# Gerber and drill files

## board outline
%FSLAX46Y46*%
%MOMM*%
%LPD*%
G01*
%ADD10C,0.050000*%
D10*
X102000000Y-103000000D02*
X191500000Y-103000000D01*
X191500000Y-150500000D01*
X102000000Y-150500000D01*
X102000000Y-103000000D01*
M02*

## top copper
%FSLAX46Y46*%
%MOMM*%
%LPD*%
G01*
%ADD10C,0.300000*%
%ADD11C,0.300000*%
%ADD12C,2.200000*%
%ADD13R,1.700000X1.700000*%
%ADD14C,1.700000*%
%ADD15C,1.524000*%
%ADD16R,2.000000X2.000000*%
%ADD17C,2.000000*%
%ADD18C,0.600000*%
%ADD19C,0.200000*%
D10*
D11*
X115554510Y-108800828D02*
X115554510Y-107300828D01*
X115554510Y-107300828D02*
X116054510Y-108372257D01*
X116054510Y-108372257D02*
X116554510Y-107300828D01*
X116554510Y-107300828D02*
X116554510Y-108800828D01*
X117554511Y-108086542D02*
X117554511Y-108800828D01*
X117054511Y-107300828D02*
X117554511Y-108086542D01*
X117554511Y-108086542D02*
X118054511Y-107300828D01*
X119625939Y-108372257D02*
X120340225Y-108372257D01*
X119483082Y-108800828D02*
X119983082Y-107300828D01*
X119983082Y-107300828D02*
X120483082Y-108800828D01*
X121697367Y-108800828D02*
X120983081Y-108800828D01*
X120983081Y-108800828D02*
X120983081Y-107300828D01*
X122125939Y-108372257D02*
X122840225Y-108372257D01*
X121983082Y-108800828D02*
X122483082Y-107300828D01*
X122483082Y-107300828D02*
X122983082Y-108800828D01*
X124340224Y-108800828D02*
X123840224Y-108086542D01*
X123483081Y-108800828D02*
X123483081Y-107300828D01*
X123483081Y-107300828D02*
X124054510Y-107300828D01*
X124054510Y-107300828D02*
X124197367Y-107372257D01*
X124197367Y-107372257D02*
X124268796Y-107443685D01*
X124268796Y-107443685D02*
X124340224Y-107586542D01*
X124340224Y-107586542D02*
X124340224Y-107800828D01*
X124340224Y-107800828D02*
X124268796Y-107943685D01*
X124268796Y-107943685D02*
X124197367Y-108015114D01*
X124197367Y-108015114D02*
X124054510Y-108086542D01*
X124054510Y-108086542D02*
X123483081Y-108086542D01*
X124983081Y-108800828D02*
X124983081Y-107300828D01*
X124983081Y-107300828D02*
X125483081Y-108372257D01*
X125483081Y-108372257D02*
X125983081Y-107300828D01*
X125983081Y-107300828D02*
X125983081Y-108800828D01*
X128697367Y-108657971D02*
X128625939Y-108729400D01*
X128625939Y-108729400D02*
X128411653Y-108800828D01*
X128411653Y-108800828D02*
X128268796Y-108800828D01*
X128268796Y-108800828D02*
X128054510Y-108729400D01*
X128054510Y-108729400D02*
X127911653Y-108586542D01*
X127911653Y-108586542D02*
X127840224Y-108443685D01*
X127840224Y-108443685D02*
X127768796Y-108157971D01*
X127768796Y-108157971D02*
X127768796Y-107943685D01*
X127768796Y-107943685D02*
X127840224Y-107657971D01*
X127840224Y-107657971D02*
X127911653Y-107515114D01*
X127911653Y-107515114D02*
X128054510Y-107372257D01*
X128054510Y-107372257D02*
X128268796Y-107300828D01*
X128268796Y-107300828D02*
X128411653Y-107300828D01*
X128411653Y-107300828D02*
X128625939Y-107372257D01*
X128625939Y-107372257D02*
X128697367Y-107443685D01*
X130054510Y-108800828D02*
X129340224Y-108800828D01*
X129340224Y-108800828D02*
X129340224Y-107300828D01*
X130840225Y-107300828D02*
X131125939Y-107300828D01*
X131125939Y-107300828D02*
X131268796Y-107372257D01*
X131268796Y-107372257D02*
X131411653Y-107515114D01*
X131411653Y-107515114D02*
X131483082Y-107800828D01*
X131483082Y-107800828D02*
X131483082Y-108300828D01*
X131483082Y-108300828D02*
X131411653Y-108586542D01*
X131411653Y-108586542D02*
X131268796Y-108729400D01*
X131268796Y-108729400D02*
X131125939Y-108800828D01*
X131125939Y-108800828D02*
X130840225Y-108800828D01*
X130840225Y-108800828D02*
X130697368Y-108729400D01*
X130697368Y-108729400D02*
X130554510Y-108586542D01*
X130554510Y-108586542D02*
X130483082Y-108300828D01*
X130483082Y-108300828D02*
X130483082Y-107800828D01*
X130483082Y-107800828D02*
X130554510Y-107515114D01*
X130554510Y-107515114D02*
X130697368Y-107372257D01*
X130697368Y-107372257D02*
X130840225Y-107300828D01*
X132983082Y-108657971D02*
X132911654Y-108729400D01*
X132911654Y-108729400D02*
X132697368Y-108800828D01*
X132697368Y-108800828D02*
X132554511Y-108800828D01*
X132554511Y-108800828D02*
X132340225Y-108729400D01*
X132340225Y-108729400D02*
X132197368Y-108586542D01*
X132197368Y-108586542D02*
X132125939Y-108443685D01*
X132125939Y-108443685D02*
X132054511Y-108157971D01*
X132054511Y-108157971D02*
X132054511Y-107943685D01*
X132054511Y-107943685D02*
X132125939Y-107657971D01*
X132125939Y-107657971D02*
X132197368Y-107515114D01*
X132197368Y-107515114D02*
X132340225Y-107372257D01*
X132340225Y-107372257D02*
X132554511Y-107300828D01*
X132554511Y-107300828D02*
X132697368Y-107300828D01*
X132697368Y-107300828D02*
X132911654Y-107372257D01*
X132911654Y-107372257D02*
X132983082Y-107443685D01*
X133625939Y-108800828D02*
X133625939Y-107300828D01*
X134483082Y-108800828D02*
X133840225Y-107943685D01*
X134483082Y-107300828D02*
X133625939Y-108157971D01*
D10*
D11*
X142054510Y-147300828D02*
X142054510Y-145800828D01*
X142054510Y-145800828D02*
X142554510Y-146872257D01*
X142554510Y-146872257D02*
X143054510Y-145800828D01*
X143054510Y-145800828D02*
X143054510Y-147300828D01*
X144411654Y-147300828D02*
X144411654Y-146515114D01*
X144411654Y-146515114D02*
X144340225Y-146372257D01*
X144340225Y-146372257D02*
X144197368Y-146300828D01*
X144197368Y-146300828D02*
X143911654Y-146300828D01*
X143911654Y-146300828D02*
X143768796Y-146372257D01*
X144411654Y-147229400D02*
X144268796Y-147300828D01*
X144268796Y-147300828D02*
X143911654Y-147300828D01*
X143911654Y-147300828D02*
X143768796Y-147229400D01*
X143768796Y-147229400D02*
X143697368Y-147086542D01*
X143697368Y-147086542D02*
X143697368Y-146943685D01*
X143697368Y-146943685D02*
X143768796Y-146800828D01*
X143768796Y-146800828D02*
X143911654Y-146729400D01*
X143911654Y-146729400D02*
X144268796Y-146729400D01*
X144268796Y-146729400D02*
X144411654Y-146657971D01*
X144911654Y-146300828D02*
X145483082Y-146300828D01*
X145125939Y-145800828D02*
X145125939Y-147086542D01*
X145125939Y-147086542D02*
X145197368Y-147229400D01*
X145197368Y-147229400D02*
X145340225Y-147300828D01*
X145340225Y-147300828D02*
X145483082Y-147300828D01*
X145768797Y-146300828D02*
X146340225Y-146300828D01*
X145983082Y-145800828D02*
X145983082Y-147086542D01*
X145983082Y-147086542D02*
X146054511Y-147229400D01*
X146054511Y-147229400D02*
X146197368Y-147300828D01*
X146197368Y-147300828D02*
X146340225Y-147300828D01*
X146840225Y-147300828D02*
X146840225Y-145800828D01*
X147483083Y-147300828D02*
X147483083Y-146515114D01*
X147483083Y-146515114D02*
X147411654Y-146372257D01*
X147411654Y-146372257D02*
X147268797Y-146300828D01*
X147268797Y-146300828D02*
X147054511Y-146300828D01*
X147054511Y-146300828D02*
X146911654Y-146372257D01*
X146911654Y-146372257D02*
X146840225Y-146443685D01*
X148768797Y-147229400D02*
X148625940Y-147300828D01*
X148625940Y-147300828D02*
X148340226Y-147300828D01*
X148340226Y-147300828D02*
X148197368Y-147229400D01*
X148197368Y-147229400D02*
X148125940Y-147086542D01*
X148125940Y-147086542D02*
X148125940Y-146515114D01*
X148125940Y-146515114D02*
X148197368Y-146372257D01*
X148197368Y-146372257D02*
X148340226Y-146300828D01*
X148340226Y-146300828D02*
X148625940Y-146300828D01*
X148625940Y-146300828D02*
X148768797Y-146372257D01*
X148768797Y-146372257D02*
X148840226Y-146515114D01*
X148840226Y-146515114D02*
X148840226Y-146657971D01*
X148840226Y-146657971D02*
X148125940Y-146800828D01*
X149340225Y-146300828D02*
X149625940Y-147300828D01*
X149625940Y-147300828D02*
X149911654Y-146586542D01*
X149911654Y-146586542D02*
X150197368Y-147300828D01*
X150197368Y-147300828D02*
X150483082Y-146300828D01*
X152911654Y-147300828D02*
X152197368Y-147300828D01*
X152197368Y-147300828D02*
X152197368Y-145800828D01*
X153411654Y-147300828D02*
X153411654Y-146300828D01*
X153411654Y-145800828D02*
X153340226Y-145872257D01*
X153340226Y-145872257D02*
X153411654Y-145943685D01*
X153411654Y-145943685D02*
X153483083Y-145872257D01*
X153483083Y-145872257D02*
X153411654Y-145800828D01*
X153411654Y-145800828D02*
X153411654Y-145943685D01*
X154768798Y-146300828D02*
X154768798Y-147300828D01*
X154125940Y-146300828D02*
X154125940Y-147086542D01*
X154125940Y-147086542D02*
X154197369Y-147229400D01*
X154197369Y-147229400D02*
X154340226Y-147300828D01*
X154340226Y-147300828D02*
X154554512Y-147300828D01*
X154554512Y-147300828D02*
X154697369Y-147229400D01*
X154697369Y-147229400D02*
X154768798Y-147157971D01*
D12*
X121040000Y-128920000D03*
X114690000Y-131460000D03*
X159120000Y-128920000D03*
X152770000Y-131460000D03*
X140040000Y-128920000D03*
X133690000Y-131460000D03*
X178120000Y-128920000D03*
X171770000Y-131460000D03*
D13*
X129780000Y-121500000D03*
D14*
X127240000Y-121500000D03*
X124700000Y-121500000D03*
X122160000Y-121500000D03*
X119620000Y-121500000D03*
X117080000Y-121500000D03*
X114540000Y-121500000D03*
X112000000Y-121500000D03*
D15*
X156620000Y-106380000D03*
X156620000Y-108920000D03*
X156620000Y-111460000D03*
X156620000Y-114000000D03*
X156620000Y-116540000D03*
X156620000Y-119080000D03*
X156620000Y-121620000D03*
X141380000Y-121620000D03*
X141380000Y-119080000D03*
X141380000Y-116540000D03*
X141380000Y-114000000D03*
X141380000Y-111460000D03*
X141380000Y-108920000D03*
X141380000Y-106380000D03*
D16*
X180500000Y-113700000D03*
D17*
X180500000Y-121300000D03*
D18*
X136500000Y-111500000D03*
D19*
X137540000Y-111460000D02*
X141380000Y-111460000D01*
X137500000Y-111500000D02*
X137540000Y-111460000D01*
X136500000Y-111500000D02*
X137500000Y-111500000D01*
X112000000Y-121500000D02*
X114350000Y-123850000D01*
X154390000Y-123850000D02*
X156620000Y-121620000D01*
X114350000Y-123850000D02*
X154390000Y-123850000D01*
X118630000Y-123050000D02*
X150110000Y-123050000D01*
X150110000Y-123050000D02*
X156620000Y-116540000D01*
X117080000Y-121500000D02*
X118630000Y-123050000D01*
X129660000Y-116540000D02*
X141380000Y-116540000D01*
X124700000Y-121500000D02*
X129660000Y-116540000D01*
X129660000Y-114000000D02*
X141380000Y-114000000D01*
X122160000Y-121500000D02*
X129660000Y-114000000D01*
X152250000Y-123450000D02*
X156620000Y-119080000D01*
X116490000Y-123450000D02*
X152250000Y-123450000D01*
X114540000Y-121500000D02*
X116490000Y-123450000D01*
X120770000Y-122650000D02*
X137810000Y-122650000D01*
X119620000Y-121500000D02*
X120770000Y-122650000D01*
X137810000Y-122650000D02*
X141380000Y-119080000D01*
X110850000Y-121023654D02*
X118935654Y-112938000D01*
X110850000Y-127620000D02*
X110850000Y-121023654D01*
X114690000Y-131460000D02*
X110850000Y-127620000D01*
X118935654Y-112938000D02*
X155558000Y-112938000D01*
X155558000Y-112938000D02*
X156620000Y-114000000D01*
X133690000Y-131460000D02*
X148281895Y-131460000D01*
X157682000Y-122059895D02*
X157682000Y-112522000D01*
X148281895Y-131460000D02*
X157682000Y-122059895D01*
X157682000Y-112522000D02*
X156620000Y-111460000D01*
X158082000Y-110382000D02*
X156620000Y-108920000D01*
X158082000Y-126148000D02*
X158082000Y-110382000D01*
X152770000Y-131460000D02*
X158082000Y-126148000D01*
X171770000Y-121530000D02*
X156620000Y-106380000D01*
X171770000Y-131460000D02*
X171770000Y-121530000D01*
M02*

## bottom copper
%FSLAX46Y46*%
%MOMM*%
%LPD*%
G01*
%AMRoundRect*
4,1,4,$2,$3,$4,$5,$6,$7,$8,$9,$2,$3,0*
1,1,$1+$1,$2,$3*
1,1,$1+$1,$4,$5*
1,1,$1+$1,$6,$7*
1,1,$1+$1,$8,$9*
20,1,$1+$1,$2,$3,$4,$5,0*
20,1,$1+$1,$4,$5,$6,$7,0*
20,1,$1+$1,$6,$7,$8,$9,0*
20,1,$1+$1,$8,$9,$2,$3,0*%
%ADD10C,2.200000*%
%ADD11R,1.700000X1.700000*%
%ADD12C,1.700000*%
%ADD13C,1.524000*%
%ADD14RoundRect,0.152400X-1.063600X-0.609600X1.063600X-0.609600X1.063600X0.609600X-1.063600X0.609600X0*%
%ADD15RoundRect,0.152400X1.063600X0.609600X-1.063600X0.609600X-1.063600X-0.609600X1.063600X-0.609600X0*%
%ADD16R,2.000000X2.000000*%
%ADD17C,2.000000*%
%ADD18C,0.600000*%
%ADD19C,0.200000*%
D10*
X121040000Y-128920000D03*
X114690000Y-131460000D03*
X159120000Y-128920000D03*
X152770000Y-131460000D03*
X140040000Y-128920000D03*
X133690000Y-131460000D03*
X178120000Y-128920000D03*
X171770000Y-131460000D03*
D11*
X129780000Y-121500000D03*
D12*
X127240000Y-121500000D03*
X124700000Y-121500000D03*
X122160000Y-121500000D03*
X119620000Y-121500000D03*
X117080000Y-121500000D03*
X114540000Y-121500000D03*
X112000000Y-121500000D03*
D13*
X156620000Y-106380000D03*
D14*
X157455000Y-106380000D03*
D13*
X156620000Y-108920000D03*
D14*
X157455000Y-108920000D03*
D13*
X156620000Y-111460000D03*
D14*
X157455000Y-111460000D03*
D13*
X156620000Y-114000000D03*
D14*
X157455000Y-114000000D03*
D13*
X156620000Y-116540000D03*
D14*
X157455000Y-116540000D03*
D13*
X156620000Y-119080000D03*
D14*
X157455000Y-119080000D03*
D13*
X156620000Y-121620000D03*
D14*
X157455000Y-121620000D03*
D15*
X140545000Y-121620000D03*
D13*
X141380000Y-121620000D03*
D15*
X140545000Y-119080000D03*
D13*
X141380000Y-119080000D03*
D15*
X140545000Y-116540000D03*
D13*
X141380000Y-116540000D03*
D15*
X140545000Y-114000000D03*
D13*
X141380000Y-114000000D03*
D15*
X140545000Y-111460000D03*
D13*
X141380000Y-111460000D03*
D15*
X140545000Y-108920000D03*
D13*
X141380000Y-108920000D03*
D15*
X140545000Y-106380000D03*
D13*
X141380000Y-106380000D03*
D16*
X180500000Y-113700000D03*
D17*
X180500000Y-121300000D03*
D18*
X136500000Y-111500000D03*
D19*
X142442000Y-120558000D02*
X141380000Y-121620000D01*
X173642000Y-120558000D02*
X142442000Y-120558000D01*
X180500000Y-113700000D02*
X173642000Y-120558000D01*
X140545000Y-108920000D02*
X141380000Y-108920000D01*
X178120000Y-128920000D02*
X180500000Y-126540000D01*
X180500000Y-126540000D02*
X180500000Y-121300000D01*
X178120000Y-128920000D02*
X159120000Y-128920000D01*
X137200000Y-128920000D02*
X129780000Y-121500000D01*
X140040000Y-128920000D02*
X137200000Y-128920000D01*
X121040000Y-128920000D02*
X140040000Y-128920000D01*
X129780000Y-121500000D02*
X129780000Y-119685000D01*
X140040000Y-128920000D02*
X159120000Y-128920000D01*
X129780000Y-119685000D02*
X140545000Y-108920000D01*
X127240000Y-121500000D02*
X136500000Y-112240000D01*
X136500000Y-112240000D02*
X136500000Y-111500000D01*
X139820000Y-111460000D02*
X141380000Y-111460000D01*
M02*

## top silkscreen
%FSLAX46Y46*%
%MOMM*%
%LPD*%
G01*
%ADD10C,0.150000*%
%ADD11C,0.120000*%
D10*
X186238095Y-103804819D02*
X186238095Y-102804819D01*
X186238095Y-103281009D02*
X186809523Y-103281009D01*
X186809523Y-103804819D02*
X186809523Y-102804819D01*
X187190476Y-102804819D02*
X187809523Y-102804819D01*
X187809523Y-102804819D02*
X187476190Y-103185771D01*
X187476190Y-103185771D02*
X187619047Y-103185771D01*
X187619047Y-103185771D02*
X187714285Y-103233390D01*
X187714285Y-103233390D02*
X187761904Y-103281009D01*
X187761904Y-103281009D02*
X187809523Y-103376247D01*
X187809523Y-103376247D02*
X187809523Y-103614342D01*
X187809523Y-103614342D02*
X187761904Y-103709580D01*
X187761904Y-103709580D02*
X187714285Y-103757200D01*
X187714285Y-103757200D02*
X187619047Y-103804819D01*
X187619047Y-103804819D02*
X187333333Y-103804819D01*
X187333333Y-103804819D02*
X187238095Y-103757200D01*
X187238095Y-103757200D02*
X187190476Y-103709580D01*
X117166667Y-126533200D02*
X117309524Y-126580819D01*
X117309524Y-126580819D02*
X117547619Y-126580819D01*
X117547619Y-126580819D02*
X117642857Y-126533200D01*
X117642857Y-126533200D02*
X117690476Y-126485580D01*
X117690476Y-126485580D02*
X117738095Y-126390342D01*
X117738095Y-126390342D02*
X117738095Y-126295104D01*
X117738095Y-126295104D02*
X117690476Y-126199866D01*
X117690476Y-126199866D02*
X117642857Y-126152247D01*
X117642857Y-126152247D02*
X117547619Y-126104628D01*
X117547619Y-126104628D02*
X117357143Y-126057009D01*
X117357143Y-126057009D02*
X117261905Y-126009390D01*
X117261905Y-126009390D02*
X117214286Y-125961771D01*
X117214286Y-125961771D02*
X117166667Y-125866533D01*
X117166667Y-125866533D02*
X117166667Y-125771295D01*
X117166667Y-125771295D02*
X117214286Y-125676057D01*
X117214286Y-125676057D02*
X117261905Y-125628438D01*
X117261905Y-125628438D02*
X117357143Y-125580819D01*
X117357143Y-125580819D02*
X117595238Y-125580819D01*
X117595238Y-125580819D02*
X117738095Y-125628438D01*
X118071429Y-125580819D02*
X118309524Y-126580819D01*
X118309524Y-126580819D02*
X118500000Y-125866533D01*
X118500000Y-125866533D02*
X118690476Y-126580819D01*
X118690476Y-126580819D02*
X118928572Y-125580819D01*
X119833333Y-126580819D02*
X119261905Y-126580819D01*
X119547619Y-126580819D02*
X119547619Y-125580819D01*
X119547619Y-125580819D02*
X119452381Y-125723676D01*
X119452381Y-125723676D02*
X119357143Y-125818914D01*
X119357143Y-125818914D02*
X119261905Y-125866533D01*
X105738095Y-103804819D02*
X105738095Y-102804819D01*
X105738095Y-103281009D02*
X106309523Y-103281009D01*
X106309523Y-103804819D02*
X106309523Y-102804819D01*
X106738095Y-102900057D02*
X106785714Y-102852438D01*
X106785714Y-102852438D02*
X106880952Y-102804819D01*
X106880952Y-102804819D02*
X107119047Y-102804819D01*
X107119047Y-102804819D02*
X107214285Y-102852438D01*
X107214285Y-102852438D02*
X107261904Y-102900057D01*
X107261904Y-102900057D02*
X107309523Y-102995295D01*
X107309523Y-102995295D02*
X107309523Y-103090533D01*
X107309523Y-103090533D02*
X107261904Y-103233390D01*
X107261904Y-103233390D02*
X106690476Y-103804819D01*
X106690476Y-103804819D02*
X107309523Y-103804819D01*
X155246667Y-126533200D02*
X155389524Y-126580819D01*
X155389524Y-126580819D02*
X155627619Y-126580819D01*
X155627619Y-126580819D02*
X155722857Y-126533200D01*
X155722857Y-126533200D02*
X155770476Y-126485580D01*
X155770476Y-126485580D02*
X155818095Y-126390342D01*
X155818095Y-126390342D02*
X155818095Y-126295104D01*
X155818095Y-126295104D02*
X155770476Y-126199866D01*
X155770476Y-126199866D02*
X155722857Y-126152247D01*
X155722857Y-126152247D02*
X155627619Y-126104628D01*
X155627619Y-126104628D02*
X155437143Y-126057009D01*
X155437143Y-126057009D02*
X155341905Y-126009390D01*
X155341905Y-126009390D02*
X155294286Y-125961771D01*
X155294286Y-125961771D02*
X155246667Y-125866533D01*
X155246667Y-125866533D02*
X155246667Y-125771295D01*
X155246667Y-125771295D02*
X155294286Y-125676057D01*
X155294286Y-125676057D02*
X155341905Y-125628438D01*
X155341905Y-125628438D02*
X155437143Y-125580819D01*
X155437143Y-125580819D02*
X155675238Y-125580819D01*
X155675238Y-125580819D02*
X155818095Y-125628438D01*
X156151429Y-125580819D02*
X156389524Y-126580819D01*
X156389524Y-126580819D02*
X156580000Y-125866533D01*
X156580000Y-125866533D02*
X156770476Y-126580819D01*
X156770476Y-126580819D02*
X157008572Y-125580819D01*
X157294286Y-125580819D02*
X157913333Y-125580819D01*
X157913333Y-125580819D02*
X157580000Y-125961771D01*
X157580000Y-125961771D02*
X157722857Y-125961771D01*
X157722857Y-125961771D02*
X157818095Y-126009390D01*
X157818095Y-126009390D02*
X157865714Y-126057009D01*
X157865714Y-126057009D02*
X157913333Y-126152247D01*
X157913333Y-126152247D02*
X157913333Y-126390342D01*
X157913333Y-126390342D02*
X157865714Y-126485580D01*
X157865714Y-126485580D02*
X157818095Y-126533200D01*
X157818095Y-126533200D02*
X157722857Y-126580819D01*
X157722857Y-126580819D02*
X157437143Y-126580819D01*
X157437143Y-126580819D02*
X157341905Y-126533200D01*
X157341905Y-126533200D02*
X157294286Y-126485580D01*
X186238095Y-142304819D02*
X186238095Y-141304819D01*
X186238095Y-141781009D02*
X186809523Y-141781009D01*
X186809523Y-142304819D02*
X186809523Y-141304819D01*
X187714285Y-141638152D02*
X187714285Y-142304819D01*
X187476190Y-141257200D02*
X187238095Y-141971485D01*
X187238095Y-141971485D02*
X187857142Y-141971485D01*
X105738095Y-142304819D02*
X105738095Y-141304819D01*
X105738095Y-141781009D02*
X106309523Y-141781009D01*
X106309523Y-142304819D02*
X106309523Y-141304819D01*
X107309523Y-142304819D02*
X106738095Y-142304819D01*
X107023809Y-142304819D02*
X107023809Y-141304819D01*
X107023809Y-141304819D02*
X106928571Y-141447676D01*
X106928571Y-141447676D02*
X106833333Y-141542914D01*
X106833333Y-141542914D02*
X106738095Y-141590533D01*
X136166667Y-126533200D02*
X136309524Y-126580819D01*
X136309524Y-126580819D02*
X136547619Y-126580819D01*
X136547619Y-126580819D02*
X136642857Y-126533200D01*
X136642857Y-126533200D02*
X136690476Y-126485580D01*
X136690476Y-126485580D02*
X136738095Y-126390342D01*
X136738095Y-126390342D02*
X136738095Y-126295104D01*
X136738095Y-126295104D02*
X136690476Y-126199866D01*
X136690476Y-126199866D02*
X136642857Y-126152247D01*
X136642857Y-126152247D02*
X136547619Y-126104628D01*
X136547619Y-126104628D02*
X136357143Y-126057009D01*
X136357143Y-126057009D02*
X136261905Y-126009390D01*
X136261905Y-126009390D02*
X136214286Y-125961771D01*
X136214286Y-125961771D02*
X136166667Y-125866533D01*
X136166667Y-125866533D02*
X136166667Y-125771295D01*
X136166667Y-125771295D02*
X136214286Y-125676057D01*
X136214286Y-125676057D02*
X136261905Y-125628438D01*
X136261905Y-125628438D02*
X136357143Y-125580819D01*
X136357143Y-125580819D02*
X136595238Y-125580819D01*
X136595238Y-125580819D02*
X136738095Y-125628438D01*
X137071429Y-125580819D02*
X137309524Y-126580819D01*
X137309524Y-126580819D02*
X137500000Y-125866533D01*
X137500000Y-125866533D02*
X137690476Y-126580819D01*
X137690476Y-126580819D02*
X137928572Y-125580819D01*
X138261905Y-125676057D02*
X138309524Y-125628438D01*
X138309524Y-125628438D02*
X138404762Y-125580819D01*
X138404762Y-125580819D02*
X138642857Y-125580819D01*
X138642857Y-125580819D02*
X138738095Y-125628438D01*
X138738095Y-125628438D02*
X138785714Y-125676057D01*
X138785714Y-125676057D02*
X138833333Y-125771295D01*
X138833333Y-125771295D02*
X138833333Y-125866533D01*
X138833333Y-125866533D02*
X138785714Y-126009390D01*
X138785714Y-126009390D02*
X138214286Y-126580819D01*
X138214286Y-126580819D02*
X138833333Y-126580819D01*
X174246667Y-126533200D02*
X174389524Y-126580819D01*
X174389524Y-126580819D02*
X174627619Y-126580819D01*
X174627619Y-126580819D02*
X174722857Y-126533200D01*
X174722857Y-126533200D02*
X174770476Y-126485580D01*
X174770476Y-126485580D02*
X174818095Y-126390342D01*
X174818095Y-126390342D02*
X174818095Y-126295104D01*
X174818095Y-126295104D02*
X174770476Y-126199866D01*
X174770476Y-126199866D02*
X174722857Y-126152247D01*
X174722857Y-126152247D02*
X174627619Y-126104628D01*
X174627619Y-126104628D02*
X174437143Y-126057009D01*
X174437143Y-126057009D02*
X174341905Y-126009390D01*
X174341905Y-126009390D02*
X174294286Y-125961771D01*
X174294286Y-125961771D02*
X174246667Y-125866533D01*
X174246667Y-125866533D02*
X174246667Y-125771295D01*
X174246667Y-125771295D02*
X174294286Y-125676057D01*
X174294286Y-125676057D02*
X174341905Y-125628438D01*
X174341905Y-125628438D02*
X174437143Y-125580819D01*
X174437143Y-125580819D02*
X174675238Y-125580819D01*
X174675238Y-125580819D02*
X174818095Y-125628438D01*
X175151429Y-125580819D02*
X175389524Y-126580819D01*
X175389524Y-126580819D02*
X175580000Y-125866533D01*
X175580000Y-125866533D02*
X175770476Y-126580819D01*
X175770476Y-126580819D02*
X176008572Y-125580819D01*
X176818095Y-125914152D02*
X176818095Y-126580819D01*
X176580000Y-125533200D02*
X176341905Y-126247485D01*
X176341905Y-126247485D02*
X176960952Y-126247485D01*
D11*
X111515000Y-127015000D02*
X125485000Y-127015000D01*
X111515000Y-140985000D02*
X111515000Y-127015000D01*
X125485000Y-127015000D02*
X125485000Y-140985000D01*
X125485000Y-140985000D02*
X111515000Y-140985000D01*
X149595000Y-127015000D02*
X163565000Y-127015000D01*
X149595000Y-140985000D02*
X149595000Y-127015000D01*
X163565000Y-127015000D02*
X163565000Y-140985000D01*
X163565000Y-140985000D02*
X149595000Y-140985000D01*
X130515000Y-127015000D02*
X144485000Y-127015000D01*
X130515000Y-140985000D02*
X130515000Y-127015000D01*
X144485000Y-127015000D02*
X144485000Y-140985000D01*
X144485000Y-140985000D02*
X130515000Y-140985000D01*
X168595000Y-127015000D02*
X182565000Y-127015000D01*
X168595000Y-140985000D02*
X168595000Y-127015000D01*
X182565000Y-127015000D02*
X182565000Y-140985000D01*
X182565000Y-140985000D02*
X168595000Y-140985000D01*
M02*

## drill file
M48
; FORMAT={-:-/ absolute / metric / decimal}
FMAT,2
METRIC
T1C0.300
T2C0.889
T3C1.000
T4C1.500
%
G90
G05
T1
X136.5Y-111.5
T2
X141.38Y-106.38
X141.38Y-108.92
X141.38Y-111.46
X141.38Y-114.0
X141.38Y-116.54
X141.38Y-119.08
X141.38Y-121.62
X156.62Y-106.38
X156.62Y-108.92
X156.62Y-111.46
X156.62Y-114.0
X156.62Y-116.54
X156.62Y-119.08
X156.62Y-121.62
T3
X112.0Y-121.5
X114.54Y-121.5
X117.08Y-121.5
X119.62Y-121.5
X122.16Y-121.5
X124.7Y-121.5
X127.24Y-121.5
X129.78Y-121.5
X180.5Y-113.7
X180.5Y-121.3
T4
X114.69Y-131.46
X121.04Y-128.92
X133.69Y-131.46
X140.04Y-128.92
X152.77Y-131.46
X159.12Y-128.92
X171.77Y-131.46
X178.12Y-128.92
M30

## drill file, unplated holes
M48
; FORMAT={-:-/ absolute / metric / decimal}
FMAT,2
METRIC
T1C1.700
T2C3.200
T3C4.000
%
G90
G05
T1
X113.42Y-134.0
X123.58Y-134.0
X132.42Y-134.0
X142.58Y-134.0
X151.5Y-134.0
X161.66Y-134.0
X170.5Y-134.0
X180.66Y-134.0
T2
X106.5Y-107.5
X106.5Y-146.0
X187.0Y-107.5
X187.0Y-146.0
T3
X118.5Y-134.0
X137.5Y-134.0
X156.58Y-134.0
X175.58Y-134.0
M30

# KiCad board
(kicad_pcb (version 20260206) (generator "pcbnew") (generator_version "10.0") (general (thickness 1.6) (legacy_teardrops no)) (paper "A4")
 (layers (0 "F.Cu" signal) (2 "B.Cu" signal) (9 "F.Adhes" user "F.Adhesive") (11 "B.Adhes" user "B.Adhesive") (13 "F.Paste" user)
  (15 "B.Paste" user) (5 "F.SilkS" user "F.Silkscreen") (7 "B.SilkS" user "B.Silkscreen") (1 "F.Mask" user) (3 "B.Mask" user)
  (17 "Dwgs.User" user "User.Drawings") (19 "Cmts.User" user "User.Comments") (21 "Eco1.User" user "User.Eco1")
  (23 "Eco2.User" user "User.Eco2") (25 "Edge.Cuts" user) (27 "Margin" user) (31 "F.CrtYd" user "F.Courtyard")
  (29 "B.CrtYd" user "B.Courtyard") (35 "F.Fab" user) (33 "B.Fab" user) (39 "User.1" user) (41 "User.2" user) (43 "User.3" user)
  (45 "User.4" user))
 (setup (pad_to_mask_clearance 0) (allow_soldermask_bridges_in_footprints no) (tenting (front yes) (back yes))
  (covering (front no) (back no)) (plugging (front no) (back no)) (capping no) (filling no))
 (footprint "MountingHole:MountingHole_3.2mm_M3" (layer "F.Cu") (at 187 107.5)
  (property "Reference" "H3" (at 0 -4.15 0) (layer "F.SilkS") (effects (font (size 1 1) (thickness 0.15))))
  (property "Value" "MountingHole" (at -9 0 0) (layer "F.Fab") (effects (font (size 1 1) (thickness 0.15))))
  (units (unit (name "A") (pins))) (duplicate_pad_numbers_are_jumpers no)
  (pad "" np_thru_hole circle (at 0 0) (size 3.2 3.2) (drill 3.2) (layers "*.Cu" "*.Mask")))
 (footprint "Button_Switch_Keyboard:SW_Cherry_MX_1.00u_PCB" (layer "F.Cu") (at 121.04 128.92)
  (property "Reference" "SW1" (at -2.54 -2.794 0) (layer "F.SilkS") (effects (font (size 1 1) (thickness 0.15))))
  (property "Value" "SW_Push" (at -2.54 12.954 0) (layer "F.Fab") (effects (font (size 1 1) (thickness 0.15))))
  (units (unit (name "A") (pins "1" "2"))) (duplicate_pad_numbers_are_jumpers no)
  (fp_line (start -9.525 -1.905) (end 4.445 -1.905) (stroke (width 0.12) (type solid)) (layer "F.SilkS"))
  (fp_line (start -9.525 12.065) (end -9.525 -1.905) (stroke (width 0.12) (type solid)) (layer "F.SilkS"))
  (fp_line (start 4.445 -1.905) (end 4.445 12.065) (stroke (width 0.12) (type solid)) (layer "F.SilkS"))
  (fp_line (start 4.445 12.065) (end -9.525 12.065) (stroke (width 0.12) (type solid)) (layer "F.SilkS"))
  (pad "" np_thru_hole circle (at -7.62 5.08) (size 1.7 1.7) (drill 1.7) (layers "*.Cu" "*.Mask"))
  (pad "" np_thru_hole circle (at -2.54 5.08) (size 4 4) (drill 4) (layers "*.Cu" "*.Mask"))
  (pad "" np_thru_hole circle (at 2.54 5.08) (size 1.7 1.7) (drill 1.7) (layers "*.Cu" "*.Mask"))
  (pad "1" thru_hole circle (at 0 0) (size 2.2 2.2) (drill 1.5) (layers "*.Cu" "*.Mask") (remove_unused_layers no) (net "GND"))
  (pad "2" thru_hole circle (at -6.35 2.54) (size 2.2 2.2) (drill 1.5) (layers "*.Cu" "*.Mask") (remove_unused_layers no)
   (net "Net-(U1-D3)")))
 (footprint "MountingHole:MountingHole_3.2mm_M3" (layer "F.Cu") (at 106.5 107.5)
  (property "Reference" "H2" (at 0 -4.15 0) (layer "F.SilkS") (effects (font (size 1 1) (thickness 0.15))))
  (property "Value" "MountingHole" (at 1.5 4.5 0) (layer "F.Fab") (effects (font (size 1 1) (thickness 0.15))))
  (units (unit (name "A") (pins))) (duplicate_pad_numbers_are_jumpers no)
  (pad "" np_thru_hole circle (at 0 0) (size 3.2 3.2) (drill 3.2) (layers "*.Cu" "*.Mask")))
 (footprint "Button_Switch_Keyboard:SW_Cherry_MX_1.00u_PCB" (layer "F.Cu") (at 159.12 128.92)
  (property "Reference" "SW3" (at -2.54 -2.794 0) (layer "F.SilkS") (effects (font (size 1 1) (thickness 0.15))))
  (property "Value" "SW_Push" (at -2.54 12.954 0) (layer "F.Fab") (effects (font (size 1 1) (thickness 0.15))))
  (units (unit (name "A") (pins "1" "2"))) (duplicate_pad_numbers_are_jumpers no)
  (fp_line (start -9.525 -1.905) (end 4.445 -1.905) (stroke (width 0.12) (type solid)) (layer "F.SilkS"))
  (fp_line (start -9.525 12.065) (end -9.525 -1.905) (stroke (width 0.12) (type solid)) (layer "F.SilkS"))
  (fp_line (start 4.445 -1.905) (end 4.445 12.065) (stroke (width 0.12) (type solid)) (layer "F.SilkS"))
  (fp_line (start 4.445 12.065) (end -9.525 12.065) (stroke (width 0.12) (type solid)) (layer "F.SilkS"))
  (pad "" np_thru_hole circle (at -7.62 5.08) (size 1.7 1.7) (drill 1.7) (layers "*.Cu" "*.Mask"))
  (pad "" np_thru_hole circle (at -2.54 5.08) (size 4 4) (drill 4) (layers "*.Cu" "*.Mask"))
  (pad "" np_thru_hole circle (at 2.54 5.08) (size 1.7 1.7) (drill 1.7) (layers "*.Cu" "*.Mask"))
  (pad "1" thru_hole circle (at 0 0) (size 2.2 2.2) (drill 1.5) (layers "*.Cu" "*.Mask") (remove_unused_layers no) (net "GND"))
  (pad "2" thru_hole circle (at -6.35 2.54) (size 2.2 2.2) (drill 1.5) (layers "*.Cu" "*.Mask") (remove_unused_layers no)
   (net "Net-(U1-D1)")))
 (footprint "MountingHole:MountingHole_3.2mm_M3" (layer "F.Cu") (at 187 146)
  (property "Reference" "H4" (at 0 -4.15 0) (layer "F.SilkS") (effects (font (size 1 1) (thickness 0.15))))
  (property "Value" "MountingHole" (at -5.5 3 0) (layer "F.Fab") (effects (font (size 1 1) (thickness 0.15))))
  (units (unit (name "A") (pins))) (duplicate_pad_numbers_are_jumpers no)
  (pad "" np_thru_hole circle (at 0 0) (size 3.2 3.2) (drill 3.2) (layers "*.Cu" "*.Mask")))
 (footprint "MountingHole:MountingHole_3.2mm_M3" (layer "F.Cu") (at 106.5 146)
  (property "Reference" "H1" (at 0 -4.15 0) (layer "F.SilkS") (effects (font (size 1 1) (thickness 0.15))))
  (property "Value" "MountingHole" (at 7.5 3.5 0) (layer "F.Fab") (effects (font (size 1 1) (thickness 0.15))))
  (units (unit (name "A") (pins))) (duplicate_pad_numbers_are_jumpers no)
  (pad "" np_thru_hole circle (at 0 0) (size 3.2 3.2) (drill 3.2) (layers "*.Cu" "*.Mask")))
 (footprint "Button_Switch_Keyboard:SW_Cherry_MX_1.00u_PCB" (layer "F.Cu") (at 140.04 128.92)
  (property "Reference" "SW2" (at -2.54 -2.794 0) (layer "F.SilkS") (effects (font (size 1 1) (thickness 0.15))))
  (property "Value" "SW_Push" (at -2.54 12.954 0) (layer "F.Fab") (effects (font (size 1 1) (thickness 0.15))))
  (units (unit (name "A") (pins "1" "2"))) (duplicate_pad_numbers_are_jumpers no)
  (fp_line (start -9.525 -1.905) (end 4.445 -1.905) (stroke (width 0.12) (type solid)) (layer "F.SilkS"))
  (fp_line (start -9.525 12.065) (end -9.525 -1.905) (stroke (width 0.12) (type solid)) (layer "F.SilkS"))
  (fp_line (start 4.445 -1.905) (end 4.445 12.065) (stroke (width 0.12) (type solid)) (layer "F.SilkS"))
  (fp_line (start 4.445 12.065) (end -9.525 12.065) (stroke (width 0.12) (type solid)) (layer "F.SilkS"))
  (pad "" np_thru_hole circle (at -7.62 5.08) (size 1.7 1.7) (drill 1.7) (layers "*.Cu" "*.Mask"))
  (pad "" np_thru_hole circle (at -2.54 5.08) (size 4 4) (drill 4) (layers "*.Cu" "*.Mask"))
  (pad "" np_thru_hole circle (at 2.54 5.08) (size 1.7 1.7) (drill 1.7) (layers "*.Cu" "*.Mask"))
  (pad "1" thru_hole circle (at 0 0) (size 2.2 2.2) (drill 1.5) (layers "*.Cu" "*.Mask") (remove_unused_layers no) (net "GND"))
  (pad "2" thru_hole circle (at -6.35 2.54) (size 2.2 2.2) (drill 1.5) (layers "*.Cu" "*.Mask") (remove_unused_layers no)
   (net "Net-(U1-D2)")))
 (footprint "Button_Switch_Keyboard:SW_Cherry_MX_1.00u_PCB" (layer "F.Cu") (at 178.12 128.92)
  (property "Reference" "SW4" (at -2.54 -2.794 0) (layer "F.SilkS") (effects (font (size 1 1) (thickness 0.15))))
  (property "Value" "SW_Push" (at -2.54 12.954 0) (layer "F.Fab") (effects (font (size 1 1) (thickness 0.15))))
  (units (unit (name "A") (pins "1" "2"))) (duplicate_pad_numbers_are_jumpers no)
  (fp_line (start -9.525 -1.905) (end 4.445 -1.905) (stroke (width 0.12) (type solid)) (layer "F.SilkS"))
  (fp_line (start -9.525 12.065) (end -9.525 -1.905) (stroke (width 0.12) (type solid)) (layer "F.SilkS"))
  (fp_line (start 4.445 -1.905) (end 4.445 12.065) (stroke (width 0.12) (type solid)) (layer "F.SilkS"))
  (fp_line (start 4.445 12.065) (end -9.525 12.065) (stroke (width 0.12) (type solid)) (layer "F.SilkS"))
  (pad "" np_thru_hole circle (at -7.62 5.08) (size 1.7 1.7) (drill 1.7) (layers "*.Cu" "*.Mask"))
  (pad "" np_thru_hole circle (at -2.54 5.08) (size 4 4) (drill 4) (layers "*.Cu" "*.Mask"))
  (pad "" np_thru_hole circle (at 2.54 5.08) (size 1.7 1.7) (drill 1.7) (layers "*.Cu" "*.Mask"))
  (pad "1" thru_hole circle (at 0 0) (size 2.2 2.2) (drill 1.5) (layers "*.Cu" "*.Mask") (remove_unused_layers no) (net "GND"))
  (pad "2" thru_hole circle (at -6.35 2.54) (size 2.2 2.2) (drill 1.5) (layers "*.Cu" "*.Mask") (remove_unused_layers no)
   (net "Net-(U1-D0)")))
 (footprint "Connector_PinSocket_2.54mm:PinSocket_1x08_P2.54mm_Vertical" (layer "B.Cu") (at 129.78 121.5 90)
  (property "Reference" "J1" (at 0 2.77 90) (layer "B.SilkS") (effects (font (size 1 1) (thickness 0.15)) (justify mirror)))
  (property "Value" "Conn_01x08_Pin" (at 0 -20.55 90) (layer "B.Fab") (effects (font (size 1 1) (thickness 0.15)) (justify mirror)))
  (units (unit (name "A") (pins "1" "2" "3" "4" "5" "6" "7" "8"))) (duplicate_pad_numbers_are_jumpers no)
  (pad "1" thru_hole rect (at 0 0 90) (size 1.7 1.7) (drill 1) (layers "*.Cu" "*.Mask") (remove_unused_layers no) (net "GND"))
  (pad "2" thru_hole circle (at 0 -2.54 90) (size 1.7 1.7) (drill 1) (layers "*.Cu" "*.Mask") (remove_unused_layers no) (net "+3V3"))
  (pad "3" thru_hole circle (at 0 -5.08 90) (size 1.7 1.7) (drill 1) (layers "*.Cu" "*.Mask") (remove_unused_layers no) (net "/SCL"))
  (pad "4" thru_hole circle (at 0 -7.62 90) (size 1.7 1.7) (drill 1) (layers "*.Cu" "*.Mask") (remove_unused_layers no) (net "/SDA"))
  (pad "5" thru_hole circle (at 0 -10.16 90) (size 1.7 1.7) (drill 1) (layers "*.Cu" "*.Mask") (remove_unused_layers no) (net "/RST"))
  (pad "6" thru_hole circle (at 0 -12.7 90) (size 1.7 1.7) (drill 1) (layers "*.Cu" "*.Mask") (remove_unused_layers no) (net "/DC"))
  (pad "7" thru_hole circle (at 0 -15.24 90) (size 1.7 1.7) (drill 1) (layers "*.Cu" "*.Mask") (remove_unused_layers no) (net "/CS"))
  (pad "8" thru_hole circle (at 0 -17.78 90) (size 1.7 1.7) (drill 1) (layers "*.Cu" "*.Mask") (remove_unused_layers no) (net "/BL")))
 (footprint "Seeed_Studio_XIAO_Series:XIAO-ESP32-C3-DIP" (layer "B.Cu") (at 149 114 90)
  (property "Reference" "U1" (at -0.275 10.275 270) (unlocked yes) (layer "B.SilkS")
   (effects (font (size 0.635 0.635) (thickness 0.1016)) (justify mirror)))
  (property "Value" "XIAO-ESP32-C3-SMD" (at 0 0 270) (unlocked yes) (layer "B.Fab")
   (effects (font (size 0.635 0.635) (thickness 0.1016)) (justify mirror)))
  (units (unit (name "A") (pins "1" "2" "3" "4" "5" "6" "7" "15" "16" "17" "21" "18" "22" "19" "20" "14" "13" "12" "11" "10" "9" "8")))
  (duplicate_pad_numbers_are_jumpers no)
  (pad "1" thru_hole circle (at 7.62 7.62) (size 1.524 1.524) (drill 0.889) (layers "*.Cu" "*.Mask") (remove_unused_layers no)
   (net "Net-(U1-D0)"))
  (pad "1" smd roundrect (at 7.62 8.455) (size 2.432 1.524) (layers "B.Cu" "B.Mask") (roundrect_rratio 0.1) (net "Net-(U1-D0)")
   (thermal_bridge_angle 45))
  (pad "2" thru_hole circle (at 5.08 7.62) (size 1.524 1.524) (drill 0.889) (layers "*.Cu" "*.Mask") (remove_unused_layers no)
   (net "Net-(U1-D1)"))
  (pad "2" smd roundrect (at 5.08 8.455) (size 2.432 1.524) (layers "B.Cu" "B.Mask") (roundrect_rratio 0.1) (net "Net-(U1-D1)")
   (thermal_bridge_angle 45))
  (pad "3" thru_hole circle (at 2.54 7.62) (size 1.524 1.524) (drill 0.889) (layers "*.Cu" "*.Mask") (remove_unused_layers no)
   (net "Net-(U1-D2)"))
  (pad "3" smd roundrect (at 2.54 8.455) (size 2.432 1.524) (layers "B.Cu" "B.Mask") (roundrect_rratio 0.1) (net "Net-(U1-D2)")
   (thermal_bridge_angle 45))
  (pad "4" thru_hole circle (at 0 7.62) (size 1.524 1.524) (drill 0.889) (layers "*.Cu" "*.Mask") (remove_unused_layers no)
   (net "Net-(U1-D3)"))
  (pad "4" smd roundrect (at 0 8.455) (size 2.432 1.524) (layers "B.Cu" "B.Mask") (roundrect_rratio 0.1) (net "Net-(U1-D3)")
   (thermal_bridge_angle 45))
  (pad "5" thru_hole circle (at -2.54 7.62) (size 1.524 1.524) (drill 0.889) (layers "*.Cu" "*.Mask") (remove_unused_layers no) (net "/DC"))
  (pad "5" smd roundrect (at -2.54 8.455) (size 2.432 1.524) (layers "B.Cu" "B.Mask") (roundrect_rratio 0.1) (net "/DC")
   (thermal_bridge_angle 45))
  (pad "6" thru_hole circle (at -5.08 7.62) (size 1.524 1.524) (drill 0.889) (layers "*.Cu" "*.Mask") (remove_unused_layers no) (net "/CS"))
  (pad "6" smd roundrect (at -5.08 8.455) (size 2.432 1.524) (layers "B.Cu" "B.Mask") (roundrect_rratio 0.1) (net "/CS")
   (thermal_bridge_angle 45))
  (pad "7" thru_hole circle (at -7.62 7.62) (size 1.524 1.524) (drill 0.889) (layers "*.Cu" "*.Mask") (remove_unused_layers no) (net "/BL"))
  (pad "7" smd roundrect (at -7.62 8.455) (size 2.432 1.524) (layers "B.Cu" "B.Mask") (roundrect_rratio 0.1) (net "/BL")
   (thermal_bridge_angle 45))
  (pad "8" smd roundrect (at -7.62 -8.455 180) (size 2.432 1.524) (layers "B.Cu" "B.Mask") (roundrect_rratio 0.1) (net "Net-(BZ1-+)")
   (thermal_bridge_angle 45))
  (pad "8" thru_hole circle (at -7.62 -7.62 180) (size 1.524 1.524) (drill 0.889) (layers "*.Cu" "*.Mask") (remove_unused_layers no)
   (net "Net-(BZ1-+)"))
  (pad "9" smd roundrect (at -5.08 -8.455 180) (size 2.432 1.524) (layers "B.Cu" "B.Mask") (roundrect_rratio 0.1) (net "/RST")
   (thermal_bridge_angle 45))
  (pad "9" thru_hole circle (at -5.08 -7.62 180) (size 1.524 1.524) (drill 0.889) (layers "*.Cu" "*.Mask") (remove_unused_layers no)
   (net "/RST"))
  (pad "10" smd roundrect (at -2.54 -8.455 180) (size 2.432 1.524) (layers "B.Cu" "B.Mask") (roundrect_rratio 0.1) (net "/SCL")
   (thermal_bridge_angle 45))
  (pad "10" thru_hole circle (at -2.54 -7.62 180) (size 1.524 1.524) (drill 0.889) (layers "*.Cu" "*.Mask") (remove_unused_layers no)
   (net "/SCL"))
  (pad "11" smd roundrect (at 0 -8.455 180) (size 2.432 1.524) (layers "B.Cu" "B.Mask") (roundrect_rratio 0.1) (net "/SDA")
   (thermal_bridge_angle 45))
  (pad "11" thru_hole circle (at 0 -7.62 180) (size 1.524 1.524) (drill 0.889) (layers "*.Cu" "*.Mask") (remove_unused_layers no)
   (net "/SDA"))
  (pad "12" smd roundrect (at 2.54 -8.455 180) (size 2.432 1.524) (layers "B.Cu" "B.Mask") (roundrect_rratio 0.1) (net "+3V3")
   (thermal_bridge_angle 45))
  (pad "12" thru_hole circle (at 2.54 -7.62 180) (size 1.524 1.524) (drill 0.889) (layers "*.Cu" "*.Mask") (remove_unused_layers no)
   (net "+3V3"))
  (pad "13" smd roundrect (at 5.08 -8.455 180) (size 2.432 1.524) (layers "B.Cu" "B.Mask") (roundrect_rratio 0.1) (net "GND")
   (thermal_bridge_angle 45))
  (pad "13" thru_hole circle (at 5.08 -7.62 180) (size 1.524 1.524) (drill 0.889) (layers "*.Cu" "*.Mask") (remove_unused_layers no)
   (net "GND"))
  (pad "14" smd roundrect (at 7.62 -8.455 180) (size 2.432 1.524) (layers "B.Cu" "B.Mask") (roundrect_rratio 0.1)
   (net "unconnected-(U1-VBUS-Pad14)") (thermal_bridge_angle 45))
  (pad "14" thru_hole circle (at 7.62 -7.62 180) (size 1.524 1.524) (drill 0.889) (layers "*.Cu" "*.Mask") (remove_unused_layers no)
   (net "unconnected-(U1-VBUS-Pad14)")))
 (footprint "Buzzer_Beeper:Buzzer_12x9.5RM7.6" (layer "B.Cu") (at 180.5 113.7 -90)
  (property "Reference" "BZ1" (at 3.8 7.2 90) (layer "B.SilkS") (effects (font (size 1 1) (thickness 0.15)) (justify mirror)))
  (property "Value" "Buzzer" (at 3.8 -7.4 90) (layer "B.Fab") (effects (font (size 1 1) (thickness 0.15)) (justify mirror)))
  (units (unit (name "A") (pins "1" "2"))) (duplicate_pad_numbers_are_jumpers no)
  (pad "1" thru_hole rect (at 0 0 270) (size 2 2) (drill 1) (layers "*.Cu" "*.Mask") (remove_unused_layers no) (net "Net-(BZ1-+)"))
  (pad "2" thru_hole circle (at 7.6 0 270) (size 2 2) (drill 1) (layers "*.Cu" "*.Mask") (remove_unused_layers no) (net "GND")))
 (gr_rect (start 102 103) (end 191.5 150.5) (stroke (width 0.05) (type default)) (fill no) (layer "Edge.Cuts"))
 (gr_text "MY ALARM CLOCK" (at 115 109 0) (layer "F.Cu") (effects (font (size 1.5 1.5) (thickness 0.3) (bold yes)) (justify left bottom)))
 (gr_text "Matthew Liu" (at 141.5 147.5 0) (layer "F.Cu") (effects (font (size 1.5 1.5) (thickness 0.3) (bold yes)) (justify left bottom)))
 (segment (start 140.545 108.92) (end 141.38 108.92) (width 0.2) (layer "B.Cu") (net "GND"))
 (segment (start 178.12 128.92) (end 180.5 126.54) (width 0.2) (layer "B.Cu") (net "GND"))
 (segment (start 180.5 126.54) (end 180.5 121.3) (width 0.2) (layer "B.Cu") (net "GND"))
 (segment (start 178.12 128.92) (end 159.12 128.92) (width 0.2) (layer "B.Cu") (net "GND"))
 (segment (start 137.2 128.92) (end 129.78 121.5) (width 0.2) (layer "B.Cu") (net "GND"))
 (segment (start 140.04 128.92) (end 137.2 128.92) (width 0.2) (layer "B.Cu") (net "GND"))
 (segment (start 121.04 128.92) (end 140.04 128.92) (width 0.2) (layer "B.Cu") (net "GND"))
 (segment (start 129.78 121.5) (end 129.78 119.685) (width 0.2) (layer "B.Cu") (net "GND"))
 (segment (start 140.04 128.92) (end 159.12 128.92) (width 0.2) (layer "B.Cu") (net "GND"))
 (segment (start 129.78 119.685) (end 140.545 108.92) (width 0.2) (layer "B.Cu") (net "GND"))
 (segment (start 110.85 121.023654) (end 118.935654 112.938) (width 0.2) (layer "F.Cu") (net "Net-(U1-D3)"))
 (segment (start 110.85 127.62) (end 110.85 121.023654) (width 0.2) (layer "F.Cu") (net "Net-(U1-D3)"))
 (segment (start 114.69 131.46) (end 110.85 127.62) (width 0.2) (layer "F.Cu") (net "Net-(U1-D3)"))
 (segment (start 118.935654 112.938) (end 155.558 112.938) (width 0.2) (layer "F.Cu") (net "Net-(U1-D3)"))
 (segment (start 155.558 112.938) (end 156.62 114) (width 0.2) (layer "F.Cu") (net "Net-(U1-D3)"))
 (segment (start 158.082 110.382) (end 156.62 108.92) (width 0.2) (layer "F.Cu") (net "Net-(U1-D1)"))
 (segment (start 158.082 126.148) (end 158.082 110.382) (width 0.2) (layer "F.Cu") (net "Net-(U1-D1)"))
 (segment (start 152.77 131.46) (end 158.082 126.148) (width 0.2) (layer "F.Cu") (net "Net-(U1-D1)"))
 (segment (start 133.69 131.46) (end 148.281895 131.46) (width 0.2) (layer "F.Cu") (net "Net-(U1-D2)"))
 (segment (start 157.682 122.059895) (end 157.682 112.522) (width 0.2) (layer "F.Cu") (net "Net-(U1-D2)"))
 (segment (start 148.281895 131.46) (end 157.682 122.059895) (width 0.2) (layer "F.Cu") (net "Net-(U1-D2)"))
 (segment (start 157.682 112.522) (end 156.62 111.46) (width 0.2) (layer "F.Cu") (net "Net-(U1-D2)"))
 (segment (start 171.77 121.53) (end 156.62 106.38) (width 0.2) (layer "F.Cu") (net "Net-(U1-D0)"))
 (segment (start 171.77 131.46) (end 171.77 121.53) (width 0.2) (layer "F.Cu") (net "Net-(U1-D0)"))
 (segment (start 137.54 111.46) (end 141.38 111.46) (width 0.2) (layer "F.Cu") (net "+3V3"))
 (segment (start 137.5 111.5) (end 137.54 111.46) (width 0.2) (layer "F.Cu") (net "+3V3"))
 (segment (start 136.5 111.5) (end 137.5 111.5) (width 0.2) (layer "F.Cu") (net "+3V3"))
 (via (at 136.5 111.5) (size 0.6) (drill 0.3) (layers "F.Cu" "B.Cu") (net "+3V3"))
 (segment (start 127.24 121.5) (end 136.5 112.24) (width 0.2) (layer "B.Cu") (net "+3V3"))
 (segment (start 136.5 112.24) (end 136.5 111.5) (width 0.2) (layer "B.Cu") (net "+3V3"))
 (segment (start 139.82 111.46) (end 141.38 111.46) (width 0.2) (layer "B.Cu") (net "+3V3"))
 (segment (start 129.66 116.54) (end 141.38 116.54) (width 0.2) (layer "F.Cu") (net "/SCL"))
 (segment (start 124.7 121.5) (end 129.66 116.54) (width 0.2) (layer "F.Cu") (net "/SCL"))
 (segment (start 129.66 114) (end 141.38 114) (width 0.2) (layer "F.Cu") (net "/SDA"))
 (segment (start 122.16 121.5) (end 129.66 114) (width 0.2) (layer "F.Cu") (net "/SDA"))
 (segment (start 120.77 122.65) (end 137.81 122.65) (width 0.2) (layer "F.Cu") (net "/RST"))
 (segment (start 119.62 121.5) (end 120.77 122.65) (width 0.2) (layer "F.Cu") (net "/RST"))
 (segment (start 137.81 122.65) (end 141.38 119.08) (width 0.2) (layer "F.Cu") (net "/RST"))
 (segment (start 118.63 123.05) (end 150.11 123.05) (width 0.2) (layer "F.Cu") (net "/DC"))
 (segment (start 150.11 123.05) (end 156.62 116.54) (width 0.2) (layer "F.Cu") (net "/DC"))
 (segment (start 117.08 121.5) (end 118.63 123.05) (width 0.2) (layer "F.Cu") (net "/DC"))
 (segment (start 152.25 123.45) (end 156.62 119.08) (width 0.2) (layer "F.Cu") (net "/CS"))
 (segment (start 116.49 123.45) (end 152.25 123.45) (width 0.2) (layer "F.Cu") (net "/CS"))
 (segment (start 114.54 121.5) (end 116.49 123.45) (width 0.2) (layer "F.Cu") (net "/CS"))
 (segment (start 112 121.5) (end 114.35 123.85) (width 0.2) (layer "F.Cu") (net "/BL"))
 (segment (start 154.39 123.85) (end 156.62 121.62) (width 0.2) (layer "F.Cu") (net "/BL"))
 (segment (start 114.35 123.85) (end 154.39 123.85) (width 0.2) (layer "F.Cu") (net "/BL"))
 (segment (start 180.5 113.7) (end 173.642 120.558) (width 0.2) (layer "B.Cu") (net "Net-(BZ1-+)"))
 (segment (start 142.442 120.558) (end 141.38 121.62) (width 0.2) (layer "B.Cu") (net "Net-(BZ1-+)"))
 (segment (start 173.642 120.558) (end 142.442 120.558) (width 0.2) (layer "B.Cu") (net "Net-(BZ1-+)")))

